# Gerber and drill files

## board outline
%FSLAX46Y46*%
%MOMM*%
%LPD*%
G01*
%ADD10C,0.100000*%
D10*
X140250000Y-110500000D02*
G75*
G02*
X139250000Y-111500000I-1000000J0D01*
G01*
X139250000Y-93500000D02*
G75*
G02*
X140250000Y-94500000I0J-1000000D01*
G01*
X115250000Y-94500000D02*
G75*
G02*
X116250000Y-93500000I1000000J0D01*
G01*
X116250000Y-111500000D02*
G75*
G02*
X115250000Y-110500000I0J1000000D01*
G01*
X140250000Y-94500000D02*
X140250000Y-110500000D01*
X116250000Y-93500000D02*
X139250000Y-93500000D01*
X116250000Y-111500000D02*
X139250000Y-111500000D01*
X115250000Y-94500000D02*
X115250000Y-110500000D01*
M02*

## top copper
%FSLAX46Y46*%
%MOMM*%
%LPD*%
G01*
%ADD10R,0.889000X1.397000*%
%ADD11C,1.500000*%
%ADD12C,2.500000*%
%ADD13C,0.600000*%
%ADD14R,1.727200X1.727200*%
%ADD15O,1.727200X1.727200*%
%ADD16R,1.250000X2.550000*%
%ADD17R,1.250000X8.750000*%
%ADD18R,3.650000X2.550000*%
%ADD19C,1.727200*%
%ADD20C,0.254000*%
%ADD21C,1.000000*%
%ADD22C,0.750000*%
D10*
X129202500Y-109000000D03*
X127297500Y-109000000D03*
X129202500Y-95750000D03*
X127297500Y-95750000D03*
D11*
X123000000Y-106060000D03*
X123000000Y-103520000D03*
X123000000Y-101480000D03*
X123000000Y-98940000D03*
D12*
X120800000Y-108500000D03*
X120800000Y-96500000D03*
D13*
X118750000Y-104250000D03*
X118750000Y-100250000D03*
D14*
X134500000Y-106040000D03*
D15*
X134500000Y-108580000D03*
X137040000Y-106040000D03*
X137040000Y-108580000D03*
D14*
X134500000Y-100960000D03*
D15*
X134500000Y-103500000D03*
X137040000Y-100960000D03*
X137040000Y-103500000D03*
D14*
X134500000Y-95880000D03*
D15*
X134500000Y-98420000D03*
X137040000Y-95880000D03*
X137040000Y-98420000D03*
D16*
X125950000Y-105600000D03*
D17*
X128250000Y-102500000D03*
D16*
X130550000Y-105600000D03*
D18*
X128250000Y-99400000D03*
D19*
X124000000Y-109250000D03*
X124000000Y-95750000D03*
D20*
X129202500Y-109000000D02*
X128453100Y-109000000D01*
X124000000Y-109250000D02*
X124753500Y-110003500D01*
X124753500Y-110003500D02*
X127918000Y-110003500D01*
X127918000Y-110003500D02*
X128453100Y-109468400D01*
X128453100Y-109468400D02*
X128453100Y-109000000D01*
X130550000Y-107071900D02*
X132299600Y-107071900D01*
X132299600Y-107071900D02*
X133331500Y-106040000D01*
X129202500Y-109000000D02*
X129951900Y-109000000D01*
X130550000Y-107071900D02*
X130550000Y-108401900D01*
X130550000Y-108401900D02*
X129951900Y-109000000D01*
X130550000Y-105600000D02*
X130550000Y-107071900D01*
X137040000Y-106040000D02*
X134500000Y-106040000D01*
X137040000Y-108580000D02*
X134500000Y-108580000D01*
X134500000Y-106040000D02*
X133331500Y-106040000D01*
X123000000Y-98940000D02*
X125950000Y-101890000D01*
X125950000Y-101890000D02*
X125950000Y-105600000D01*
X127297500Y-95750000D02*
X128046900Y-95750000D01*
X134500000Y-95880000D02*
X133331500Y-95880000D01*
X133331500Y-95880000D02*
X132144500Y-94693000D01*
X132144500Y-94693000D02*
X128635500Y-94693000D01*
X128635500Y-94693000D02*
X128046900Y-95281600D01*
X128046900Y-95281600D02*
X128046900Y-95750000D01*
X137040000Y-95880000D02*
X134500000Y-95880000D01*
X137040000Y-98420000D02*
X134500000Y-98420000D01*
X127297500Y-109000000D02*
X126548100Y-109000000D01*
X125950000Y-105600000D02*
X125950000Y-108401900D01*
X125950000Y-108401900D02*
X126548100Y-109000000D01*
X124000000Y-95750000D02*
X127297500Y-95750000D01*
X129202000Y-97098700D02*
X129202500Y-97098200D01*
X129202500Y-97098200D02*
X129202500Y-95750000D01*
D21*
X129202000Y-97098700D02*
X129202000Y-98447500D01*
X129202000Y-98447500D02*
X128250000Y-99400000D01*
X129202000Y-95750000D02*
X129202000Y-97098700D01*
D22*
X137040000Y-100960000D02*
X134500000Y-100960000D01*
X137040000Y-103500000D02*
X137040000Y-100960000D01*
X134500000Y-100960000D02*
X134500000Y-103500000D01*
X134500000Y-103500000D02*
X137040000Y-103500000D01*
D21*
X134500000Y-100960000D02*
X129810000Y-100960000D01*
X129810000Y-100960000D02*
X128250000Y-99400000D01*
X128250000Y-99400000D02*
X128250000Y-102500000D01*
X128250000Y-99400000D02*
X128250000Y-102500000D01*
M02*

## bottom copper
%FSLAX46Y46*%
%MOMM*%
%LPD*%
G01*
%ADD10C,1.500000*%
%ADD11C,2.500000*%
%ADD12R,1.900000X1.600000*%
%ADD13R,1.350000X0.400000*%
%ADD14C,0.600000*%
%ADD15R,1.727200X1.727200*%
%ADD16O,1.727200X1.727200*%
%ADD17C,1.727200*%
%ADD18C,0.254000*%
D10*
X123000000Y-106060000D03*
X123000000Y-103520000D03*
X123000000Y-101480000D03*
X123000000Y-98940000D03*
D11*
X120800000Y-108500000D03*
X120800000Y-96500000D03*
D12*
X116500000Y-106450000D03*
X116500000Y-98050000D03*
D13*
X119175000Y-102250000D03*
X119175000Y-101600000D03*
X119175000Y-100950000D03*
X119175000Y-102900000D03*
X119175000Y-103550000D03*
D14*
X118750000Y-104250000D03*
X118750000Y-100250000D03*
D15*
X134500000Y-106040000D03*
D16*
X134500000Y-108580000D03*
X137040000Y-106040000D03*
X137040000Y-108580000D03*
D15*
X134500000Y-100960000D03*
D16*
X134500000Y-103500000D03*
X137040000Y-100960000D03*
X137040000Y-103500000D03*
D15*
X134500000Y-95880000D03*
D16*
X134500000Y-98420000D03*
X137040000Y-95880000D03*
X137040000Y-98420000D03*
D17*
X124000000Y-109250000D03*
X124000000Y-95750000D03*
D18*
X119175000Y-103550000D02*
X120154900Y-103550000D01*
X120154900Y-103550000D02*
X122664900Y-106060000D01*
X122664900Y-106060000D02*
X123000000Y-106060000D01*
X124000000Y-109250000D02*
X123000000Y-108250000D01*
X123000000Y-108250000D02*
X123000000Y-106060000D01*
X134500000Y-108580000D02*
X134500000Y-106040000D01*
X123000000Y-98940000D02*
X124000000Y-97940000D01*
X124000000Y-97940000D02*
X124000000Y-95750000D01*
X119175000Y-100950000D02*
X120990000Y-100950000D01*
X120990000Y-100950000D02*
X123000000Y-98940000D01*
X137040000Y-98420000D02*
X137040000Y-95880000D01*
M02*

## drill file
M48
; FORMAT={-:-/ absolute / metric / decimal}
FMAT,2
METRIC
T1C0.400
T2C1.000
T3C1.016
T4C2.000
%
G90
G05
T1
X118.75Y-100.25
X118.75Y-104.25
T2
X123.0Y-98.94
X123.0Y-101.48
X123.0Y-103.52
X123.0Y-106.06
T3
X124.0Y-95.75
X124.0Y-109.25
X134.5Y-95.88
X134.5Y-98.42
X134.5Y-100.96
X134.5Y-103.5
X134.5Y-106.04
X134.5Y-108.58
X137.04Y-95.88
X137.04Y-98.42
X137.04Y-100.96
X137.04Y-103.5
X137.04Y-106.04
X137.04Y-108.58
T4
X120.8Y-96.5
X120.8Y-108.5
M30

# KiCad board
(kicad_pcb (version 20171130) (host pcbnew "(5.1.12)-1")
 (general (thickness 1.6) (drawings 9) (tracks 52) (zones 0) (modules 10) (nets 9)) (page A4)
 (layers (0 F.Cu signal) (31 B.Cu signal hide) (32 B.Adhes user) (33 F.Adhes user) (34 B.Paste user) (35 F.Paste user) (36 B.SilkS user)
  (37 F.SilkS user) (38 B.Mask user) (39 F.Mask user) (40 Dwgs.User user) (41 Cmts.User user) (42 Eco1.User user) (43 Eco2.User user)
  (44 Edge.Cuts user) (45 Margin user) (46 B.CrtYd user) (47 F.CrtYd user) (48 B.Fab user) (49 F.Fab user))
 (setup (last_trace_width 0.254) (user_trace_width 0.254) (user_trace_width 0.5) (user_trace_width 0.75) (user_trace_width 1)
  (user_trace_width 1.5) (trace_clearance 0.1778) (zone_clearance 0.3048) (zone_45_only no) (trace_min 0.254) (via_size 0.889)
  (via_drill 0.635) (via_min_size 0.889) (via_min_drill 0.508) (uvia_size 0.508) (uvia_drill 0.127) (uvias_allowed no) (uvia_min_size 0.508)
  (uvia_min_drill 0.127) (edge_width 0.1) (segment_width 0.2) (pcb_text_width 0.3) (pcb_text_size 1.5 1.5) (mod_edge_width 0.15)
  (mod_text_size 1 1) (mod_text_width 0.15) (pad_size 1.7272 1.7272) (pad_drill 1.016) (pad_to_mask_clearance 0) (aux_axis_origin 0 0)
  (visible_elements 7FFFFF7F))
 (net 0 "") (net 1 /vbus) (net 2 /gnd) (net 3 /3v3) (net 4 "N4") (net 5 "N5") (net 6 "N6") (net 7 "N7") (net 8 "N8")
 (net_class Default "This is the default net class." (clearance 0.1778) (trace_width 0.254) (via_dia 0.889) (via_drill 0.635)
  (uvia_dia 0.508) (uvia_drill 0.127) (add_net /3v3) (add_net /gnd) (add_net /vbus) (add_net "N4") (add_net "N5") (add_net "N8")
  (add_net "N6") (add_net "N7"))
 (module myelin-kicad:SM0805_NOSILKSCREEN (layer F.Cu) (at 128.25 109 180)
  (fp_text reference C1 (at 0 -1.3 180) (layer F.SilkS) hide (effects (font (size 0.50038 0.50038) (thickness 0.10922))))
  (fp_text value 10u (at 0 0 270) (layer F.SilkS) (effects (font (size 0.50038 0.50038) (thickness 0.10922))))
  (pad 1 smd rect (at -0.9525 0 180) (size 0.889 1.397) (layers F.Cu F.Paste F.Mask) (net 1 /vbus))
  (pad 2 smd rect (at 0.9525 0 180) (size 0.889 1.397) (layers F.Cu F.Paste F.Mask) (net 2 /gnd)))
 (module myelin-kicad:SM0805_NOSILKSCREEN (layer F.Cu) (at 128.25 95.75 180)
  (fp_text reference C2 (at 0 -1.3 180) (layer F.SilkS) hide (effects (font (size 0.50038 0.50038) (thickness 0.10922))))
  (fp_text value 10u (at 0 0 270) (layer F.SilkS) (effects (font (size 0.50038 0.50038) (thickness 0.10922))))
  (pad 1 smd rect (at -0.9525 0 180) (size 0.889 1.397) (layers F.Cu F.Paste F.Mask) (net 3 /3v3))
  (pad 2 smd rect (at 0.9525 0 180) (size 0.889 1.397) (layers F.Cu F.Paste F.Mask) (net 2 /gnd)))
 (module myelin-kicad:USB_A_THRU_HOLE (layer F.Cu) (at 115 102.5 270)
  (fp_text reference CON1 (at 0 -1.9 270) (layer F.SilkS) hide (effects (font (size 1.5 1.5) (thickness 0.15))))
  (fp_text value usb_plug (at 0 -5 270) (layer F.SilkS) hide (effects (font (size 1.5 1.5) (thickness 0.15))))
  (pad 1 thru_hole circle (at 3.56 -8 90) (size 1.5 1.5) (drill 1) (layers *.Cu *.Mask F.SilkS) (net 1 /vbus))
  (pad 2 thru_hole circle (at 1.02 -8 90) (size 1.5 1.5) (drill 1) (layers *.Cu *.Mask F.SilkS) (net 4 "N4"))
  (pad 3 thru_hole circle (at -1.02 -8 90) (size 1.5 1.5) (drill 1) (layers *.Cu *.Mask F.SilkS) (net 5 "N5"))
  (pad 4 thru_hole circle (at -3.56 -8 90) (size 1.5 1.5) (drill 1) (layers *.Cu *.Mask F.SilkS) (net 2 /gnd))
  (pad "" thru_hole circle (at 6 -5.8 90) (size 2.5 2.5) (drill 2) (layers *.Cu *.Mask F.SilkS))
  (pad "" thru_hole circle (at -6 -5.8 90) (size 2.5 2.5) (drill 2) (layers *.Cu *.Mask F.SilkS)))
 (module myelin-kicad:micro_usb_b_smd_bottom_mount (layer B.Cu) (at 116.5 102.25 90)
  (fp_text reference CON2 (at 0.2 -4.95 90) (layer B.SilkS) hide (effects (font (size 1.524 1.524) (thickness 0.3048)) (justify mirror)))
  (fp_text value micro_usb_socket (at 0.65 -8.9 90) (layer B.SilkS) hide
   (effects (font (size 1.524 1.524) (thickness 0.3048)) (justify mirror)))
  (pad "" smd rect (at -4.2 0 90) (size 1.6 1.9) (layers B.Cu B.Paste B.Mask))
  (pad "" smd rect (at 4.2 0 90) (size 1.6 1.9) (layers B.Cu B.Paste B.Mask))
  (pad 3 smd rect (at 0 2.675 90) (size 0.4 1.35) (layers B.Cu B.Paste B.Mask) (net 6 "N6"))
  (pad 4 smd rect (at 0.65 2.675 90) (size 0.4 1.35) (layers B.Cu B.Paste B.Mask) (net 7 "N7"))
  (pad 5 smd rect (at 1.3 2.675 90) (size 0.4 1.35) (layers B.Cu B.Paste B.Mask) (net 2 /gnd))
  (pad 2 smd rect (at -0.65 2.675 90) (size 0.4 1.35) (layers B.Cu B.Paste B.Mask) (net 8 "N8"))
  (pad 1 smd rect (at -1.3 2.675 90) (size 0.4 1.35) (layers B.Cu B.Paste B.Mask) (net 1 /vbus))
  (pad "" thru_hole circle (at -2 2.25 90) (size 0.6 0.6) (drill 0.4) (layers *.Cu *.Mask B.SilkS))
  (pad "" thru_hole circle (at 2 2.25 90) (size 0.6 0.6) (drill 0.4) (layers *.Cu *.Mask B.SilkS)))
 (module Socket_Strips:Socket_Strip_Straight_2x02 (layer F.Cu) (at 134.5 106.04)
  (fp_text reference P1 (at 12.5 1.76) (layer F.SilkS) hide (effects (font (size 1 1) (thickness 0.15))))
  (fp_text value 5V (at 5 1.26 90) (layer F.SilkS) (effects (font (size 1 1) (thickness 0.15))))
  (pad 1 thru_hole rect (at 0 0) (size 1.7272 1.7272) (drill 1.016) (layers *.Cu *.Mask F.SilkS) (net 1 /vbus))
  (pad 2 thru_hole oval (at 0 2.54) (size 1.7272 1.7272) (drill 1.016) (layers *.Cu *.Mask F.SilkS) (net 1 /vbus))
  (pad 3 thru_hole oval (at 2.54 0) (size 1.7272 1.7272) (drill 1.016) (layers *.Cu *.Mask F.SilkS) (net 1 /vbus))
  (pad 4 thru_hole oval (at 2.54 2.54) (size 1.7272 1.7272) (drill 1.016) (layers *.Cu *.Mask F.SilkS) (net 1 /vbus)))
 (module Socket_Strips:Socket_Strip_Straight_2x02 (layer F.Cu) (at 134.5 100.96)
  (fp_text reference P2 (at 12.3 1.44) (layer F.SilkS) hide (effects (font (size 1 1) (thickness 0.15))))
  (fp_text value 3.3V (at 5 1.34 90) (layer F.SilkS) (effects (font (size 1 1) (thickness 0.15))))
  (pad 1 thru_hole rect (at 0 0) (size 1.7272 1.7272) (drill 1.016) (layers *.Cu *.Mask F.SilkS) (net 3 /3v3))
  (pad 2 thru_hole oval (at 0 2.54) (size 1.7272 1.7272) (drill 1.016) (layers *.Cu *.Mask F.SilkS) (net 3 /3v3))
  (pad 3 thru_hole oval (at 2.54 0) (size 1.7272 1.7272) (drill 1.016) (layers *.Cu *.Mask F.SilkS) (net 3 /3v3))
  (pad 4 thru_hole oval (at 2.54 2.54) (size 1.7272 1.7272) (drill 1.016) (layers *.Cu *.Mask F.SilkS) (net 3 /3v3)))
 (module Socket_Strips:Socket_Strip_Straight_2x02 (layer F.Cu) (at 134.5 95.88)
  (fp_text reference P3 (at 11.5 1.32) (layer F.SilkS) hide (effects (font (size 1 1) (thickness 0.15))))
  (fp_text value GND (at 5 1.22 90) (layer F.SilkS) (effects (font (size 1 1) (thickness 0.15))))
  (pad 1 thru_hole rect (at 0 0) (size 1.7272 1.7272) (drill 1.016) (layers *.Cu *.Mask F.SilkS) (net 2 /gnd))
  (pad 2 thru_hole oval (at 0 2.54) (size 1.7272 1.7272) (drill 1.016) (layers *.Cu *.Mask F.SilkS) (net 2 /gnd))
  (pad 3 thru_hole oval (at 2.54 0) (size 1.7272 1.7272) (drill 1.016) (layers *.Cu *.Mask F.SilkS) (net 2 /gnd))
  (pad 4 thru_hole oval (at 2.54 2.54) (size 1.7272 1.7272) (drill 1.016) (layers *.Cu *.Mask F.SilkS) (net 2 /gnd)))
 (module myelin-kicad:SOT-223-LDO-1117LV (layer F.Cu) (at 128.25 102.5)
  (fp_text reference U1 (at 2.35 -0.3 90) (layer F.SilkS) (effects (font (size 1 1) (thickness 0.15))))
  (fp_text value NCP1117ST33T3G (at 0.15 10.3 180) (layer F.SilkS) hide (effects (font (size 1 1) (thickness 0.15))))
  (pad 1 smd rect (at -2.3 3.1) (size 1.25 2.55) (layers F.Cu F.Paste F.Mask) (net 2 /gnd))
  (pad 2 smd rect (at 0 0) (size 1.25 8.75) (layers F.Cu F.Paste F.Mask) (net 3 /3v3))
  (pad 3 smd rect (at 2.3 3.1) (size 1.25 2.55) (layers F.Cu F.Paste F.Mask) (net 1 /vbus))
  (pad 2 smd rect (at 0 -3.1) (size 3.65 2.55) (layers F.Cu F.Paste F.Mask) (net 3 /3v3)))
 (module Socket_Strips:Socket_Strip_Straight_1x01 (layer F.Cu) (at 124 109.25)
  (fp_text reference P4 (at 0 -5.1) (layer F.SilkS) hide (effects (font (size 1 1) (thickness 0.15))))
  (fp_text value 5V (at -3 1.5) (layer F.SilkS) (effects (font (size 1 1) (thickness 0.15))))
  (pad 1 thru_hole circle (at 0 0) (size 1.7272 1.7272) (drill 1.016) (layers *.Cu *.Mask F.SilkS) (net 1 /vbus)))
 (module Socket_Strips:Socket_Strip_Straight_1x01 (layer F.Cu) (at 124 95.75)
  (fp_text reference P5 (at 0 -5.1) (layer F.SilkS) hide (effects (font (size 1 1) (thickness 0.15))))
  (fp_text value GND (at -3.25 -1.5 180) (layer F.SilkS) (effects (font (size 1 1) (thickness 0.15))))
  (pad 1 thru_hole circle (at 0 0) (size 1.7272 1.7272) (drill 1.016) (layers *.Cu *.Mask F.SilkS) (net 2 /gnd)))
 (gr_arc (start 139.25 110.5) (end 140.25 110.5) (angle 90) (layer Edge.Cuts) (width 0.1))
 (gr_arc (start 139.25 94.5) (end 139.25 93.5) (angle 90) (layer Edge.Cuts) (width 0.1))
 (gr_arc (start 116.25 94.5) (end 115.25 94.5) (angle 90) (layer Edge.Cuts) (width 0.1))
 (gr_arc (start 116.25 110.5) (end 116.25 111.5) (angle 90) (layer Edge.Cuts) (width 0.1))
 (gr_line (start 140.25 94.5) (end 140.25 110.5) (angle 90) (layer Edge.Cuts) (width 0.1))
 (gr_line (start 116.25 93.5) (end 139.25 93.5) (angle 90) (layer Edge.Cuts) (width 0.1))
 (gr_line (start 116.25 111.5) (end 139.25 111.5) (angle 90) (layer Edge.Cuts) (width 0.1))
 (gr_line (start 115.25 94.5) (end 115.25 110.5) (angle 90) (layer Edge.Cuts) (width 0.1))
 (segment (start 129.2025 109) (end 128.4531 109) (width 0.254) (layer F.Cu) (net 1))
 (segment (start 124 109.25) (end 124.7535 110.0035) (width 0.254) (layer F.Cu) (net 1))
 (segment (start 124.7535 110.0035) (end 127.918 110.0035) (width 0.254) (layer F.Cu) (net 1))
 (segment (start 127.918 110.0035) (end 128.4531 109.4684) (width 0.254) (layer F.Cu) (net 1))
 (segment (start 128.4531 109.4684) (end 128.4531 109) (width 0.254) (layer F.Cu) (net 1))
 (segment (start 119.175 103.55) (end 120.1549 103.55) (width 0.254) (layer B.Cu) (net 1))
 (segment (start 120.1549 103.55) (end 122.6649 106.06) (width 0.254) (layer B.Cu) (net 1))
 (segment (start 122.6649 106.06) (end 123 106.06) (width 0.254) (layer B.Cu) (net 1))
 (segment (start 124 109.25) (end 123 108.25) (width 0.254) (layer B.Cu) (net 1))
 (segment (start 123 108.25) (end 123 106.06) (width 0.254) (layer B.Cu) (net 1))
 (segment (start 130.55 107.0719) (end 132.2996 107.0719) (width 0.254) (layer F.Cu) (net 1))
 (segment (start 132.2996 107.0719) (end 133.3315 106.04) (width 0.254) (layer F.Cu) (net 1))
 (segment (start 129.2025 109) (end 129.9519 109) (width 0.254) (layer F.Cu) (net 1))
 (segment (start 130.55 107.0719) (end 130.55 108.4019) (width 0.254) (layer F.Cu) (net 1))
 (segment (start 130.55 108.4019) (end 129.9519 109) (width 0.254) (layer F.Cu) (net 1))
 (segment (start 130.55 105.6) (end 130.55 107.0719) (width 0.254) (layer F.Cu) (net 1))
 (segment (start 134.5 108.58) (end 134.5 106.04) (width 0.254) (layer B.Cu) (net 1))
 (segment (start 137.04 106.04) (end 134.5 106.04) (width 0.254) (layer F.Cu) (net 1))
 (segment (start 137.04 108.58) (end 134.5 108.58) (width 0.254) (layer F.Cu) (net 1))
 (segment (start 134.5 106.04) (end 133.3315 106.04) (width 0.254) (layer F.Cu) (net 1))
 (segment (start 123 98.94) (end 125.95 101.89) (width 0.254) (layer F.Cu) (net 2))
 (segment (start 125.95 101.89) (end 125.95 105.6) (width 0.254) (layer F.Cu) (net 2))
 (segment (start 123 98.94) (end 124 97.94) (width 0.254) (layer B.Cu) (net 2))
 (segment (start 124 97.94) (end 124 95.75) (width 0.254) (layer B.Cu) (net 2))
 (segment (start 119.175 100.95) (end 120.99 100.95) (width 0.254) (layer B.Cu) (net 2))
 (segment (start 120.99 100.95) (end 123 98.94) (width 0.254) (layer B.Cu) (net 2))
 (segment (start 127.2975 95.75) (end 128.0469 95.75) (width 0.254) (layer F.Cu) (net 2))
 (segment (start 134.5 95.88) (end 133.3315 95.88) (width 0.254) (layer F.Cu) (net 2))
 (segment (start 133.3315 95.88) (end 132.1445 94.693) (width 0.254) (layer F.Cu) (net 2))
 (segment (start 132.1445 94.693) (end 128.6355 94.693) (width 0.254) (layer F.Cu) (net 2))
 (segment (start 128.6355 94.693) (end 128.0469 95.2816) (width 0.254) (layer F.Cu) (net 2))
 (segment (start 128.0469 95.2816) (end 128.0469 95.75) (width 0.254) (layer F.Cu) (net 2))
 (segment (start 137.04 95.88) (end 134.5 95.88) (width 0.254) (layer F.Cu) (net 2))
 (segment (start 137.04 98.42) (end 137.04 95.88) (width 0.254) (layer B.Cu) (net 2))
 (segment (start 137.04 98.42) (end 134.5 98.42) (width 0.254) (layer F.Cu) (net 2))
 (segment (start 127.2975 109) (end 126.5481 109) (width 0.254) (layer F.Cu) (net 2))
 (segment (start 125.95 105.6) (end 125.95 108.4019) (width 0.254) (layer F.Cu) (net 2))
 (segment (start 125.95 108.4019) (end 126.5481 109) (width 0.254) (layer F.Cu) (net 2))
 (segment (start 124 95.75) (end 127.2975 95.75) (width 0.254) (layer F.Cu) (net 2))
 (segment (start 129.202 97.0987) (end 129.2025 97.0982) (width 0.254) (layer F.Cu) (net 3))
 (segment (start 129.2025 97.0982) (end 129.2025 95.75) (width 0.254) (layer F.Cu) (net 3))
 (segment (start 129.202 97.0987) (end 129.202 98.4475) (width 1) (layer F.Cu) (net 3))
 (segment (start 129.202 98.4475) (end 128.25 99.4) (width 1) (layer F.Cu) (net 3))
 (segment (start 129.202 95.75) (end 129.202 97.0987) (width 1) (layer F.Cu) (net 3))
 (segment (start 137.04 100.96) (end 134.5 100.96) (width 0.75) (layer F.Cu) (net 3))
 (segment (start 137.04 103.5) (end 137.04 100.96) (width 0.75) (layer F.Cu) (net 3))
 (segment (start 134.5 100.96) (end 134.5 103.5) (width 0.75) (layer F.Cu) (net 3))
 (segment (start 134.5 103.5) (end 137.04 103.5) (width 0.75) (layer F.Cu) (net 3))
 (segment (start 134.5 100.96) (end 129.81 100.96) (width 1) (layer F.Cu) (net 3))
 (segment (start 129.81 100.96) (end 128.25 99.4) (width 1) (layer F.Cu) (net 3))
 (segment (start 128.25 99.4) (end 128.25 102.5) (width 1) (layer F.Cu) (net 3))
 (segment (start 128.25 99.4) (end 128.25 102.5) (width 1) (layer F.Cu) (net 3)))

